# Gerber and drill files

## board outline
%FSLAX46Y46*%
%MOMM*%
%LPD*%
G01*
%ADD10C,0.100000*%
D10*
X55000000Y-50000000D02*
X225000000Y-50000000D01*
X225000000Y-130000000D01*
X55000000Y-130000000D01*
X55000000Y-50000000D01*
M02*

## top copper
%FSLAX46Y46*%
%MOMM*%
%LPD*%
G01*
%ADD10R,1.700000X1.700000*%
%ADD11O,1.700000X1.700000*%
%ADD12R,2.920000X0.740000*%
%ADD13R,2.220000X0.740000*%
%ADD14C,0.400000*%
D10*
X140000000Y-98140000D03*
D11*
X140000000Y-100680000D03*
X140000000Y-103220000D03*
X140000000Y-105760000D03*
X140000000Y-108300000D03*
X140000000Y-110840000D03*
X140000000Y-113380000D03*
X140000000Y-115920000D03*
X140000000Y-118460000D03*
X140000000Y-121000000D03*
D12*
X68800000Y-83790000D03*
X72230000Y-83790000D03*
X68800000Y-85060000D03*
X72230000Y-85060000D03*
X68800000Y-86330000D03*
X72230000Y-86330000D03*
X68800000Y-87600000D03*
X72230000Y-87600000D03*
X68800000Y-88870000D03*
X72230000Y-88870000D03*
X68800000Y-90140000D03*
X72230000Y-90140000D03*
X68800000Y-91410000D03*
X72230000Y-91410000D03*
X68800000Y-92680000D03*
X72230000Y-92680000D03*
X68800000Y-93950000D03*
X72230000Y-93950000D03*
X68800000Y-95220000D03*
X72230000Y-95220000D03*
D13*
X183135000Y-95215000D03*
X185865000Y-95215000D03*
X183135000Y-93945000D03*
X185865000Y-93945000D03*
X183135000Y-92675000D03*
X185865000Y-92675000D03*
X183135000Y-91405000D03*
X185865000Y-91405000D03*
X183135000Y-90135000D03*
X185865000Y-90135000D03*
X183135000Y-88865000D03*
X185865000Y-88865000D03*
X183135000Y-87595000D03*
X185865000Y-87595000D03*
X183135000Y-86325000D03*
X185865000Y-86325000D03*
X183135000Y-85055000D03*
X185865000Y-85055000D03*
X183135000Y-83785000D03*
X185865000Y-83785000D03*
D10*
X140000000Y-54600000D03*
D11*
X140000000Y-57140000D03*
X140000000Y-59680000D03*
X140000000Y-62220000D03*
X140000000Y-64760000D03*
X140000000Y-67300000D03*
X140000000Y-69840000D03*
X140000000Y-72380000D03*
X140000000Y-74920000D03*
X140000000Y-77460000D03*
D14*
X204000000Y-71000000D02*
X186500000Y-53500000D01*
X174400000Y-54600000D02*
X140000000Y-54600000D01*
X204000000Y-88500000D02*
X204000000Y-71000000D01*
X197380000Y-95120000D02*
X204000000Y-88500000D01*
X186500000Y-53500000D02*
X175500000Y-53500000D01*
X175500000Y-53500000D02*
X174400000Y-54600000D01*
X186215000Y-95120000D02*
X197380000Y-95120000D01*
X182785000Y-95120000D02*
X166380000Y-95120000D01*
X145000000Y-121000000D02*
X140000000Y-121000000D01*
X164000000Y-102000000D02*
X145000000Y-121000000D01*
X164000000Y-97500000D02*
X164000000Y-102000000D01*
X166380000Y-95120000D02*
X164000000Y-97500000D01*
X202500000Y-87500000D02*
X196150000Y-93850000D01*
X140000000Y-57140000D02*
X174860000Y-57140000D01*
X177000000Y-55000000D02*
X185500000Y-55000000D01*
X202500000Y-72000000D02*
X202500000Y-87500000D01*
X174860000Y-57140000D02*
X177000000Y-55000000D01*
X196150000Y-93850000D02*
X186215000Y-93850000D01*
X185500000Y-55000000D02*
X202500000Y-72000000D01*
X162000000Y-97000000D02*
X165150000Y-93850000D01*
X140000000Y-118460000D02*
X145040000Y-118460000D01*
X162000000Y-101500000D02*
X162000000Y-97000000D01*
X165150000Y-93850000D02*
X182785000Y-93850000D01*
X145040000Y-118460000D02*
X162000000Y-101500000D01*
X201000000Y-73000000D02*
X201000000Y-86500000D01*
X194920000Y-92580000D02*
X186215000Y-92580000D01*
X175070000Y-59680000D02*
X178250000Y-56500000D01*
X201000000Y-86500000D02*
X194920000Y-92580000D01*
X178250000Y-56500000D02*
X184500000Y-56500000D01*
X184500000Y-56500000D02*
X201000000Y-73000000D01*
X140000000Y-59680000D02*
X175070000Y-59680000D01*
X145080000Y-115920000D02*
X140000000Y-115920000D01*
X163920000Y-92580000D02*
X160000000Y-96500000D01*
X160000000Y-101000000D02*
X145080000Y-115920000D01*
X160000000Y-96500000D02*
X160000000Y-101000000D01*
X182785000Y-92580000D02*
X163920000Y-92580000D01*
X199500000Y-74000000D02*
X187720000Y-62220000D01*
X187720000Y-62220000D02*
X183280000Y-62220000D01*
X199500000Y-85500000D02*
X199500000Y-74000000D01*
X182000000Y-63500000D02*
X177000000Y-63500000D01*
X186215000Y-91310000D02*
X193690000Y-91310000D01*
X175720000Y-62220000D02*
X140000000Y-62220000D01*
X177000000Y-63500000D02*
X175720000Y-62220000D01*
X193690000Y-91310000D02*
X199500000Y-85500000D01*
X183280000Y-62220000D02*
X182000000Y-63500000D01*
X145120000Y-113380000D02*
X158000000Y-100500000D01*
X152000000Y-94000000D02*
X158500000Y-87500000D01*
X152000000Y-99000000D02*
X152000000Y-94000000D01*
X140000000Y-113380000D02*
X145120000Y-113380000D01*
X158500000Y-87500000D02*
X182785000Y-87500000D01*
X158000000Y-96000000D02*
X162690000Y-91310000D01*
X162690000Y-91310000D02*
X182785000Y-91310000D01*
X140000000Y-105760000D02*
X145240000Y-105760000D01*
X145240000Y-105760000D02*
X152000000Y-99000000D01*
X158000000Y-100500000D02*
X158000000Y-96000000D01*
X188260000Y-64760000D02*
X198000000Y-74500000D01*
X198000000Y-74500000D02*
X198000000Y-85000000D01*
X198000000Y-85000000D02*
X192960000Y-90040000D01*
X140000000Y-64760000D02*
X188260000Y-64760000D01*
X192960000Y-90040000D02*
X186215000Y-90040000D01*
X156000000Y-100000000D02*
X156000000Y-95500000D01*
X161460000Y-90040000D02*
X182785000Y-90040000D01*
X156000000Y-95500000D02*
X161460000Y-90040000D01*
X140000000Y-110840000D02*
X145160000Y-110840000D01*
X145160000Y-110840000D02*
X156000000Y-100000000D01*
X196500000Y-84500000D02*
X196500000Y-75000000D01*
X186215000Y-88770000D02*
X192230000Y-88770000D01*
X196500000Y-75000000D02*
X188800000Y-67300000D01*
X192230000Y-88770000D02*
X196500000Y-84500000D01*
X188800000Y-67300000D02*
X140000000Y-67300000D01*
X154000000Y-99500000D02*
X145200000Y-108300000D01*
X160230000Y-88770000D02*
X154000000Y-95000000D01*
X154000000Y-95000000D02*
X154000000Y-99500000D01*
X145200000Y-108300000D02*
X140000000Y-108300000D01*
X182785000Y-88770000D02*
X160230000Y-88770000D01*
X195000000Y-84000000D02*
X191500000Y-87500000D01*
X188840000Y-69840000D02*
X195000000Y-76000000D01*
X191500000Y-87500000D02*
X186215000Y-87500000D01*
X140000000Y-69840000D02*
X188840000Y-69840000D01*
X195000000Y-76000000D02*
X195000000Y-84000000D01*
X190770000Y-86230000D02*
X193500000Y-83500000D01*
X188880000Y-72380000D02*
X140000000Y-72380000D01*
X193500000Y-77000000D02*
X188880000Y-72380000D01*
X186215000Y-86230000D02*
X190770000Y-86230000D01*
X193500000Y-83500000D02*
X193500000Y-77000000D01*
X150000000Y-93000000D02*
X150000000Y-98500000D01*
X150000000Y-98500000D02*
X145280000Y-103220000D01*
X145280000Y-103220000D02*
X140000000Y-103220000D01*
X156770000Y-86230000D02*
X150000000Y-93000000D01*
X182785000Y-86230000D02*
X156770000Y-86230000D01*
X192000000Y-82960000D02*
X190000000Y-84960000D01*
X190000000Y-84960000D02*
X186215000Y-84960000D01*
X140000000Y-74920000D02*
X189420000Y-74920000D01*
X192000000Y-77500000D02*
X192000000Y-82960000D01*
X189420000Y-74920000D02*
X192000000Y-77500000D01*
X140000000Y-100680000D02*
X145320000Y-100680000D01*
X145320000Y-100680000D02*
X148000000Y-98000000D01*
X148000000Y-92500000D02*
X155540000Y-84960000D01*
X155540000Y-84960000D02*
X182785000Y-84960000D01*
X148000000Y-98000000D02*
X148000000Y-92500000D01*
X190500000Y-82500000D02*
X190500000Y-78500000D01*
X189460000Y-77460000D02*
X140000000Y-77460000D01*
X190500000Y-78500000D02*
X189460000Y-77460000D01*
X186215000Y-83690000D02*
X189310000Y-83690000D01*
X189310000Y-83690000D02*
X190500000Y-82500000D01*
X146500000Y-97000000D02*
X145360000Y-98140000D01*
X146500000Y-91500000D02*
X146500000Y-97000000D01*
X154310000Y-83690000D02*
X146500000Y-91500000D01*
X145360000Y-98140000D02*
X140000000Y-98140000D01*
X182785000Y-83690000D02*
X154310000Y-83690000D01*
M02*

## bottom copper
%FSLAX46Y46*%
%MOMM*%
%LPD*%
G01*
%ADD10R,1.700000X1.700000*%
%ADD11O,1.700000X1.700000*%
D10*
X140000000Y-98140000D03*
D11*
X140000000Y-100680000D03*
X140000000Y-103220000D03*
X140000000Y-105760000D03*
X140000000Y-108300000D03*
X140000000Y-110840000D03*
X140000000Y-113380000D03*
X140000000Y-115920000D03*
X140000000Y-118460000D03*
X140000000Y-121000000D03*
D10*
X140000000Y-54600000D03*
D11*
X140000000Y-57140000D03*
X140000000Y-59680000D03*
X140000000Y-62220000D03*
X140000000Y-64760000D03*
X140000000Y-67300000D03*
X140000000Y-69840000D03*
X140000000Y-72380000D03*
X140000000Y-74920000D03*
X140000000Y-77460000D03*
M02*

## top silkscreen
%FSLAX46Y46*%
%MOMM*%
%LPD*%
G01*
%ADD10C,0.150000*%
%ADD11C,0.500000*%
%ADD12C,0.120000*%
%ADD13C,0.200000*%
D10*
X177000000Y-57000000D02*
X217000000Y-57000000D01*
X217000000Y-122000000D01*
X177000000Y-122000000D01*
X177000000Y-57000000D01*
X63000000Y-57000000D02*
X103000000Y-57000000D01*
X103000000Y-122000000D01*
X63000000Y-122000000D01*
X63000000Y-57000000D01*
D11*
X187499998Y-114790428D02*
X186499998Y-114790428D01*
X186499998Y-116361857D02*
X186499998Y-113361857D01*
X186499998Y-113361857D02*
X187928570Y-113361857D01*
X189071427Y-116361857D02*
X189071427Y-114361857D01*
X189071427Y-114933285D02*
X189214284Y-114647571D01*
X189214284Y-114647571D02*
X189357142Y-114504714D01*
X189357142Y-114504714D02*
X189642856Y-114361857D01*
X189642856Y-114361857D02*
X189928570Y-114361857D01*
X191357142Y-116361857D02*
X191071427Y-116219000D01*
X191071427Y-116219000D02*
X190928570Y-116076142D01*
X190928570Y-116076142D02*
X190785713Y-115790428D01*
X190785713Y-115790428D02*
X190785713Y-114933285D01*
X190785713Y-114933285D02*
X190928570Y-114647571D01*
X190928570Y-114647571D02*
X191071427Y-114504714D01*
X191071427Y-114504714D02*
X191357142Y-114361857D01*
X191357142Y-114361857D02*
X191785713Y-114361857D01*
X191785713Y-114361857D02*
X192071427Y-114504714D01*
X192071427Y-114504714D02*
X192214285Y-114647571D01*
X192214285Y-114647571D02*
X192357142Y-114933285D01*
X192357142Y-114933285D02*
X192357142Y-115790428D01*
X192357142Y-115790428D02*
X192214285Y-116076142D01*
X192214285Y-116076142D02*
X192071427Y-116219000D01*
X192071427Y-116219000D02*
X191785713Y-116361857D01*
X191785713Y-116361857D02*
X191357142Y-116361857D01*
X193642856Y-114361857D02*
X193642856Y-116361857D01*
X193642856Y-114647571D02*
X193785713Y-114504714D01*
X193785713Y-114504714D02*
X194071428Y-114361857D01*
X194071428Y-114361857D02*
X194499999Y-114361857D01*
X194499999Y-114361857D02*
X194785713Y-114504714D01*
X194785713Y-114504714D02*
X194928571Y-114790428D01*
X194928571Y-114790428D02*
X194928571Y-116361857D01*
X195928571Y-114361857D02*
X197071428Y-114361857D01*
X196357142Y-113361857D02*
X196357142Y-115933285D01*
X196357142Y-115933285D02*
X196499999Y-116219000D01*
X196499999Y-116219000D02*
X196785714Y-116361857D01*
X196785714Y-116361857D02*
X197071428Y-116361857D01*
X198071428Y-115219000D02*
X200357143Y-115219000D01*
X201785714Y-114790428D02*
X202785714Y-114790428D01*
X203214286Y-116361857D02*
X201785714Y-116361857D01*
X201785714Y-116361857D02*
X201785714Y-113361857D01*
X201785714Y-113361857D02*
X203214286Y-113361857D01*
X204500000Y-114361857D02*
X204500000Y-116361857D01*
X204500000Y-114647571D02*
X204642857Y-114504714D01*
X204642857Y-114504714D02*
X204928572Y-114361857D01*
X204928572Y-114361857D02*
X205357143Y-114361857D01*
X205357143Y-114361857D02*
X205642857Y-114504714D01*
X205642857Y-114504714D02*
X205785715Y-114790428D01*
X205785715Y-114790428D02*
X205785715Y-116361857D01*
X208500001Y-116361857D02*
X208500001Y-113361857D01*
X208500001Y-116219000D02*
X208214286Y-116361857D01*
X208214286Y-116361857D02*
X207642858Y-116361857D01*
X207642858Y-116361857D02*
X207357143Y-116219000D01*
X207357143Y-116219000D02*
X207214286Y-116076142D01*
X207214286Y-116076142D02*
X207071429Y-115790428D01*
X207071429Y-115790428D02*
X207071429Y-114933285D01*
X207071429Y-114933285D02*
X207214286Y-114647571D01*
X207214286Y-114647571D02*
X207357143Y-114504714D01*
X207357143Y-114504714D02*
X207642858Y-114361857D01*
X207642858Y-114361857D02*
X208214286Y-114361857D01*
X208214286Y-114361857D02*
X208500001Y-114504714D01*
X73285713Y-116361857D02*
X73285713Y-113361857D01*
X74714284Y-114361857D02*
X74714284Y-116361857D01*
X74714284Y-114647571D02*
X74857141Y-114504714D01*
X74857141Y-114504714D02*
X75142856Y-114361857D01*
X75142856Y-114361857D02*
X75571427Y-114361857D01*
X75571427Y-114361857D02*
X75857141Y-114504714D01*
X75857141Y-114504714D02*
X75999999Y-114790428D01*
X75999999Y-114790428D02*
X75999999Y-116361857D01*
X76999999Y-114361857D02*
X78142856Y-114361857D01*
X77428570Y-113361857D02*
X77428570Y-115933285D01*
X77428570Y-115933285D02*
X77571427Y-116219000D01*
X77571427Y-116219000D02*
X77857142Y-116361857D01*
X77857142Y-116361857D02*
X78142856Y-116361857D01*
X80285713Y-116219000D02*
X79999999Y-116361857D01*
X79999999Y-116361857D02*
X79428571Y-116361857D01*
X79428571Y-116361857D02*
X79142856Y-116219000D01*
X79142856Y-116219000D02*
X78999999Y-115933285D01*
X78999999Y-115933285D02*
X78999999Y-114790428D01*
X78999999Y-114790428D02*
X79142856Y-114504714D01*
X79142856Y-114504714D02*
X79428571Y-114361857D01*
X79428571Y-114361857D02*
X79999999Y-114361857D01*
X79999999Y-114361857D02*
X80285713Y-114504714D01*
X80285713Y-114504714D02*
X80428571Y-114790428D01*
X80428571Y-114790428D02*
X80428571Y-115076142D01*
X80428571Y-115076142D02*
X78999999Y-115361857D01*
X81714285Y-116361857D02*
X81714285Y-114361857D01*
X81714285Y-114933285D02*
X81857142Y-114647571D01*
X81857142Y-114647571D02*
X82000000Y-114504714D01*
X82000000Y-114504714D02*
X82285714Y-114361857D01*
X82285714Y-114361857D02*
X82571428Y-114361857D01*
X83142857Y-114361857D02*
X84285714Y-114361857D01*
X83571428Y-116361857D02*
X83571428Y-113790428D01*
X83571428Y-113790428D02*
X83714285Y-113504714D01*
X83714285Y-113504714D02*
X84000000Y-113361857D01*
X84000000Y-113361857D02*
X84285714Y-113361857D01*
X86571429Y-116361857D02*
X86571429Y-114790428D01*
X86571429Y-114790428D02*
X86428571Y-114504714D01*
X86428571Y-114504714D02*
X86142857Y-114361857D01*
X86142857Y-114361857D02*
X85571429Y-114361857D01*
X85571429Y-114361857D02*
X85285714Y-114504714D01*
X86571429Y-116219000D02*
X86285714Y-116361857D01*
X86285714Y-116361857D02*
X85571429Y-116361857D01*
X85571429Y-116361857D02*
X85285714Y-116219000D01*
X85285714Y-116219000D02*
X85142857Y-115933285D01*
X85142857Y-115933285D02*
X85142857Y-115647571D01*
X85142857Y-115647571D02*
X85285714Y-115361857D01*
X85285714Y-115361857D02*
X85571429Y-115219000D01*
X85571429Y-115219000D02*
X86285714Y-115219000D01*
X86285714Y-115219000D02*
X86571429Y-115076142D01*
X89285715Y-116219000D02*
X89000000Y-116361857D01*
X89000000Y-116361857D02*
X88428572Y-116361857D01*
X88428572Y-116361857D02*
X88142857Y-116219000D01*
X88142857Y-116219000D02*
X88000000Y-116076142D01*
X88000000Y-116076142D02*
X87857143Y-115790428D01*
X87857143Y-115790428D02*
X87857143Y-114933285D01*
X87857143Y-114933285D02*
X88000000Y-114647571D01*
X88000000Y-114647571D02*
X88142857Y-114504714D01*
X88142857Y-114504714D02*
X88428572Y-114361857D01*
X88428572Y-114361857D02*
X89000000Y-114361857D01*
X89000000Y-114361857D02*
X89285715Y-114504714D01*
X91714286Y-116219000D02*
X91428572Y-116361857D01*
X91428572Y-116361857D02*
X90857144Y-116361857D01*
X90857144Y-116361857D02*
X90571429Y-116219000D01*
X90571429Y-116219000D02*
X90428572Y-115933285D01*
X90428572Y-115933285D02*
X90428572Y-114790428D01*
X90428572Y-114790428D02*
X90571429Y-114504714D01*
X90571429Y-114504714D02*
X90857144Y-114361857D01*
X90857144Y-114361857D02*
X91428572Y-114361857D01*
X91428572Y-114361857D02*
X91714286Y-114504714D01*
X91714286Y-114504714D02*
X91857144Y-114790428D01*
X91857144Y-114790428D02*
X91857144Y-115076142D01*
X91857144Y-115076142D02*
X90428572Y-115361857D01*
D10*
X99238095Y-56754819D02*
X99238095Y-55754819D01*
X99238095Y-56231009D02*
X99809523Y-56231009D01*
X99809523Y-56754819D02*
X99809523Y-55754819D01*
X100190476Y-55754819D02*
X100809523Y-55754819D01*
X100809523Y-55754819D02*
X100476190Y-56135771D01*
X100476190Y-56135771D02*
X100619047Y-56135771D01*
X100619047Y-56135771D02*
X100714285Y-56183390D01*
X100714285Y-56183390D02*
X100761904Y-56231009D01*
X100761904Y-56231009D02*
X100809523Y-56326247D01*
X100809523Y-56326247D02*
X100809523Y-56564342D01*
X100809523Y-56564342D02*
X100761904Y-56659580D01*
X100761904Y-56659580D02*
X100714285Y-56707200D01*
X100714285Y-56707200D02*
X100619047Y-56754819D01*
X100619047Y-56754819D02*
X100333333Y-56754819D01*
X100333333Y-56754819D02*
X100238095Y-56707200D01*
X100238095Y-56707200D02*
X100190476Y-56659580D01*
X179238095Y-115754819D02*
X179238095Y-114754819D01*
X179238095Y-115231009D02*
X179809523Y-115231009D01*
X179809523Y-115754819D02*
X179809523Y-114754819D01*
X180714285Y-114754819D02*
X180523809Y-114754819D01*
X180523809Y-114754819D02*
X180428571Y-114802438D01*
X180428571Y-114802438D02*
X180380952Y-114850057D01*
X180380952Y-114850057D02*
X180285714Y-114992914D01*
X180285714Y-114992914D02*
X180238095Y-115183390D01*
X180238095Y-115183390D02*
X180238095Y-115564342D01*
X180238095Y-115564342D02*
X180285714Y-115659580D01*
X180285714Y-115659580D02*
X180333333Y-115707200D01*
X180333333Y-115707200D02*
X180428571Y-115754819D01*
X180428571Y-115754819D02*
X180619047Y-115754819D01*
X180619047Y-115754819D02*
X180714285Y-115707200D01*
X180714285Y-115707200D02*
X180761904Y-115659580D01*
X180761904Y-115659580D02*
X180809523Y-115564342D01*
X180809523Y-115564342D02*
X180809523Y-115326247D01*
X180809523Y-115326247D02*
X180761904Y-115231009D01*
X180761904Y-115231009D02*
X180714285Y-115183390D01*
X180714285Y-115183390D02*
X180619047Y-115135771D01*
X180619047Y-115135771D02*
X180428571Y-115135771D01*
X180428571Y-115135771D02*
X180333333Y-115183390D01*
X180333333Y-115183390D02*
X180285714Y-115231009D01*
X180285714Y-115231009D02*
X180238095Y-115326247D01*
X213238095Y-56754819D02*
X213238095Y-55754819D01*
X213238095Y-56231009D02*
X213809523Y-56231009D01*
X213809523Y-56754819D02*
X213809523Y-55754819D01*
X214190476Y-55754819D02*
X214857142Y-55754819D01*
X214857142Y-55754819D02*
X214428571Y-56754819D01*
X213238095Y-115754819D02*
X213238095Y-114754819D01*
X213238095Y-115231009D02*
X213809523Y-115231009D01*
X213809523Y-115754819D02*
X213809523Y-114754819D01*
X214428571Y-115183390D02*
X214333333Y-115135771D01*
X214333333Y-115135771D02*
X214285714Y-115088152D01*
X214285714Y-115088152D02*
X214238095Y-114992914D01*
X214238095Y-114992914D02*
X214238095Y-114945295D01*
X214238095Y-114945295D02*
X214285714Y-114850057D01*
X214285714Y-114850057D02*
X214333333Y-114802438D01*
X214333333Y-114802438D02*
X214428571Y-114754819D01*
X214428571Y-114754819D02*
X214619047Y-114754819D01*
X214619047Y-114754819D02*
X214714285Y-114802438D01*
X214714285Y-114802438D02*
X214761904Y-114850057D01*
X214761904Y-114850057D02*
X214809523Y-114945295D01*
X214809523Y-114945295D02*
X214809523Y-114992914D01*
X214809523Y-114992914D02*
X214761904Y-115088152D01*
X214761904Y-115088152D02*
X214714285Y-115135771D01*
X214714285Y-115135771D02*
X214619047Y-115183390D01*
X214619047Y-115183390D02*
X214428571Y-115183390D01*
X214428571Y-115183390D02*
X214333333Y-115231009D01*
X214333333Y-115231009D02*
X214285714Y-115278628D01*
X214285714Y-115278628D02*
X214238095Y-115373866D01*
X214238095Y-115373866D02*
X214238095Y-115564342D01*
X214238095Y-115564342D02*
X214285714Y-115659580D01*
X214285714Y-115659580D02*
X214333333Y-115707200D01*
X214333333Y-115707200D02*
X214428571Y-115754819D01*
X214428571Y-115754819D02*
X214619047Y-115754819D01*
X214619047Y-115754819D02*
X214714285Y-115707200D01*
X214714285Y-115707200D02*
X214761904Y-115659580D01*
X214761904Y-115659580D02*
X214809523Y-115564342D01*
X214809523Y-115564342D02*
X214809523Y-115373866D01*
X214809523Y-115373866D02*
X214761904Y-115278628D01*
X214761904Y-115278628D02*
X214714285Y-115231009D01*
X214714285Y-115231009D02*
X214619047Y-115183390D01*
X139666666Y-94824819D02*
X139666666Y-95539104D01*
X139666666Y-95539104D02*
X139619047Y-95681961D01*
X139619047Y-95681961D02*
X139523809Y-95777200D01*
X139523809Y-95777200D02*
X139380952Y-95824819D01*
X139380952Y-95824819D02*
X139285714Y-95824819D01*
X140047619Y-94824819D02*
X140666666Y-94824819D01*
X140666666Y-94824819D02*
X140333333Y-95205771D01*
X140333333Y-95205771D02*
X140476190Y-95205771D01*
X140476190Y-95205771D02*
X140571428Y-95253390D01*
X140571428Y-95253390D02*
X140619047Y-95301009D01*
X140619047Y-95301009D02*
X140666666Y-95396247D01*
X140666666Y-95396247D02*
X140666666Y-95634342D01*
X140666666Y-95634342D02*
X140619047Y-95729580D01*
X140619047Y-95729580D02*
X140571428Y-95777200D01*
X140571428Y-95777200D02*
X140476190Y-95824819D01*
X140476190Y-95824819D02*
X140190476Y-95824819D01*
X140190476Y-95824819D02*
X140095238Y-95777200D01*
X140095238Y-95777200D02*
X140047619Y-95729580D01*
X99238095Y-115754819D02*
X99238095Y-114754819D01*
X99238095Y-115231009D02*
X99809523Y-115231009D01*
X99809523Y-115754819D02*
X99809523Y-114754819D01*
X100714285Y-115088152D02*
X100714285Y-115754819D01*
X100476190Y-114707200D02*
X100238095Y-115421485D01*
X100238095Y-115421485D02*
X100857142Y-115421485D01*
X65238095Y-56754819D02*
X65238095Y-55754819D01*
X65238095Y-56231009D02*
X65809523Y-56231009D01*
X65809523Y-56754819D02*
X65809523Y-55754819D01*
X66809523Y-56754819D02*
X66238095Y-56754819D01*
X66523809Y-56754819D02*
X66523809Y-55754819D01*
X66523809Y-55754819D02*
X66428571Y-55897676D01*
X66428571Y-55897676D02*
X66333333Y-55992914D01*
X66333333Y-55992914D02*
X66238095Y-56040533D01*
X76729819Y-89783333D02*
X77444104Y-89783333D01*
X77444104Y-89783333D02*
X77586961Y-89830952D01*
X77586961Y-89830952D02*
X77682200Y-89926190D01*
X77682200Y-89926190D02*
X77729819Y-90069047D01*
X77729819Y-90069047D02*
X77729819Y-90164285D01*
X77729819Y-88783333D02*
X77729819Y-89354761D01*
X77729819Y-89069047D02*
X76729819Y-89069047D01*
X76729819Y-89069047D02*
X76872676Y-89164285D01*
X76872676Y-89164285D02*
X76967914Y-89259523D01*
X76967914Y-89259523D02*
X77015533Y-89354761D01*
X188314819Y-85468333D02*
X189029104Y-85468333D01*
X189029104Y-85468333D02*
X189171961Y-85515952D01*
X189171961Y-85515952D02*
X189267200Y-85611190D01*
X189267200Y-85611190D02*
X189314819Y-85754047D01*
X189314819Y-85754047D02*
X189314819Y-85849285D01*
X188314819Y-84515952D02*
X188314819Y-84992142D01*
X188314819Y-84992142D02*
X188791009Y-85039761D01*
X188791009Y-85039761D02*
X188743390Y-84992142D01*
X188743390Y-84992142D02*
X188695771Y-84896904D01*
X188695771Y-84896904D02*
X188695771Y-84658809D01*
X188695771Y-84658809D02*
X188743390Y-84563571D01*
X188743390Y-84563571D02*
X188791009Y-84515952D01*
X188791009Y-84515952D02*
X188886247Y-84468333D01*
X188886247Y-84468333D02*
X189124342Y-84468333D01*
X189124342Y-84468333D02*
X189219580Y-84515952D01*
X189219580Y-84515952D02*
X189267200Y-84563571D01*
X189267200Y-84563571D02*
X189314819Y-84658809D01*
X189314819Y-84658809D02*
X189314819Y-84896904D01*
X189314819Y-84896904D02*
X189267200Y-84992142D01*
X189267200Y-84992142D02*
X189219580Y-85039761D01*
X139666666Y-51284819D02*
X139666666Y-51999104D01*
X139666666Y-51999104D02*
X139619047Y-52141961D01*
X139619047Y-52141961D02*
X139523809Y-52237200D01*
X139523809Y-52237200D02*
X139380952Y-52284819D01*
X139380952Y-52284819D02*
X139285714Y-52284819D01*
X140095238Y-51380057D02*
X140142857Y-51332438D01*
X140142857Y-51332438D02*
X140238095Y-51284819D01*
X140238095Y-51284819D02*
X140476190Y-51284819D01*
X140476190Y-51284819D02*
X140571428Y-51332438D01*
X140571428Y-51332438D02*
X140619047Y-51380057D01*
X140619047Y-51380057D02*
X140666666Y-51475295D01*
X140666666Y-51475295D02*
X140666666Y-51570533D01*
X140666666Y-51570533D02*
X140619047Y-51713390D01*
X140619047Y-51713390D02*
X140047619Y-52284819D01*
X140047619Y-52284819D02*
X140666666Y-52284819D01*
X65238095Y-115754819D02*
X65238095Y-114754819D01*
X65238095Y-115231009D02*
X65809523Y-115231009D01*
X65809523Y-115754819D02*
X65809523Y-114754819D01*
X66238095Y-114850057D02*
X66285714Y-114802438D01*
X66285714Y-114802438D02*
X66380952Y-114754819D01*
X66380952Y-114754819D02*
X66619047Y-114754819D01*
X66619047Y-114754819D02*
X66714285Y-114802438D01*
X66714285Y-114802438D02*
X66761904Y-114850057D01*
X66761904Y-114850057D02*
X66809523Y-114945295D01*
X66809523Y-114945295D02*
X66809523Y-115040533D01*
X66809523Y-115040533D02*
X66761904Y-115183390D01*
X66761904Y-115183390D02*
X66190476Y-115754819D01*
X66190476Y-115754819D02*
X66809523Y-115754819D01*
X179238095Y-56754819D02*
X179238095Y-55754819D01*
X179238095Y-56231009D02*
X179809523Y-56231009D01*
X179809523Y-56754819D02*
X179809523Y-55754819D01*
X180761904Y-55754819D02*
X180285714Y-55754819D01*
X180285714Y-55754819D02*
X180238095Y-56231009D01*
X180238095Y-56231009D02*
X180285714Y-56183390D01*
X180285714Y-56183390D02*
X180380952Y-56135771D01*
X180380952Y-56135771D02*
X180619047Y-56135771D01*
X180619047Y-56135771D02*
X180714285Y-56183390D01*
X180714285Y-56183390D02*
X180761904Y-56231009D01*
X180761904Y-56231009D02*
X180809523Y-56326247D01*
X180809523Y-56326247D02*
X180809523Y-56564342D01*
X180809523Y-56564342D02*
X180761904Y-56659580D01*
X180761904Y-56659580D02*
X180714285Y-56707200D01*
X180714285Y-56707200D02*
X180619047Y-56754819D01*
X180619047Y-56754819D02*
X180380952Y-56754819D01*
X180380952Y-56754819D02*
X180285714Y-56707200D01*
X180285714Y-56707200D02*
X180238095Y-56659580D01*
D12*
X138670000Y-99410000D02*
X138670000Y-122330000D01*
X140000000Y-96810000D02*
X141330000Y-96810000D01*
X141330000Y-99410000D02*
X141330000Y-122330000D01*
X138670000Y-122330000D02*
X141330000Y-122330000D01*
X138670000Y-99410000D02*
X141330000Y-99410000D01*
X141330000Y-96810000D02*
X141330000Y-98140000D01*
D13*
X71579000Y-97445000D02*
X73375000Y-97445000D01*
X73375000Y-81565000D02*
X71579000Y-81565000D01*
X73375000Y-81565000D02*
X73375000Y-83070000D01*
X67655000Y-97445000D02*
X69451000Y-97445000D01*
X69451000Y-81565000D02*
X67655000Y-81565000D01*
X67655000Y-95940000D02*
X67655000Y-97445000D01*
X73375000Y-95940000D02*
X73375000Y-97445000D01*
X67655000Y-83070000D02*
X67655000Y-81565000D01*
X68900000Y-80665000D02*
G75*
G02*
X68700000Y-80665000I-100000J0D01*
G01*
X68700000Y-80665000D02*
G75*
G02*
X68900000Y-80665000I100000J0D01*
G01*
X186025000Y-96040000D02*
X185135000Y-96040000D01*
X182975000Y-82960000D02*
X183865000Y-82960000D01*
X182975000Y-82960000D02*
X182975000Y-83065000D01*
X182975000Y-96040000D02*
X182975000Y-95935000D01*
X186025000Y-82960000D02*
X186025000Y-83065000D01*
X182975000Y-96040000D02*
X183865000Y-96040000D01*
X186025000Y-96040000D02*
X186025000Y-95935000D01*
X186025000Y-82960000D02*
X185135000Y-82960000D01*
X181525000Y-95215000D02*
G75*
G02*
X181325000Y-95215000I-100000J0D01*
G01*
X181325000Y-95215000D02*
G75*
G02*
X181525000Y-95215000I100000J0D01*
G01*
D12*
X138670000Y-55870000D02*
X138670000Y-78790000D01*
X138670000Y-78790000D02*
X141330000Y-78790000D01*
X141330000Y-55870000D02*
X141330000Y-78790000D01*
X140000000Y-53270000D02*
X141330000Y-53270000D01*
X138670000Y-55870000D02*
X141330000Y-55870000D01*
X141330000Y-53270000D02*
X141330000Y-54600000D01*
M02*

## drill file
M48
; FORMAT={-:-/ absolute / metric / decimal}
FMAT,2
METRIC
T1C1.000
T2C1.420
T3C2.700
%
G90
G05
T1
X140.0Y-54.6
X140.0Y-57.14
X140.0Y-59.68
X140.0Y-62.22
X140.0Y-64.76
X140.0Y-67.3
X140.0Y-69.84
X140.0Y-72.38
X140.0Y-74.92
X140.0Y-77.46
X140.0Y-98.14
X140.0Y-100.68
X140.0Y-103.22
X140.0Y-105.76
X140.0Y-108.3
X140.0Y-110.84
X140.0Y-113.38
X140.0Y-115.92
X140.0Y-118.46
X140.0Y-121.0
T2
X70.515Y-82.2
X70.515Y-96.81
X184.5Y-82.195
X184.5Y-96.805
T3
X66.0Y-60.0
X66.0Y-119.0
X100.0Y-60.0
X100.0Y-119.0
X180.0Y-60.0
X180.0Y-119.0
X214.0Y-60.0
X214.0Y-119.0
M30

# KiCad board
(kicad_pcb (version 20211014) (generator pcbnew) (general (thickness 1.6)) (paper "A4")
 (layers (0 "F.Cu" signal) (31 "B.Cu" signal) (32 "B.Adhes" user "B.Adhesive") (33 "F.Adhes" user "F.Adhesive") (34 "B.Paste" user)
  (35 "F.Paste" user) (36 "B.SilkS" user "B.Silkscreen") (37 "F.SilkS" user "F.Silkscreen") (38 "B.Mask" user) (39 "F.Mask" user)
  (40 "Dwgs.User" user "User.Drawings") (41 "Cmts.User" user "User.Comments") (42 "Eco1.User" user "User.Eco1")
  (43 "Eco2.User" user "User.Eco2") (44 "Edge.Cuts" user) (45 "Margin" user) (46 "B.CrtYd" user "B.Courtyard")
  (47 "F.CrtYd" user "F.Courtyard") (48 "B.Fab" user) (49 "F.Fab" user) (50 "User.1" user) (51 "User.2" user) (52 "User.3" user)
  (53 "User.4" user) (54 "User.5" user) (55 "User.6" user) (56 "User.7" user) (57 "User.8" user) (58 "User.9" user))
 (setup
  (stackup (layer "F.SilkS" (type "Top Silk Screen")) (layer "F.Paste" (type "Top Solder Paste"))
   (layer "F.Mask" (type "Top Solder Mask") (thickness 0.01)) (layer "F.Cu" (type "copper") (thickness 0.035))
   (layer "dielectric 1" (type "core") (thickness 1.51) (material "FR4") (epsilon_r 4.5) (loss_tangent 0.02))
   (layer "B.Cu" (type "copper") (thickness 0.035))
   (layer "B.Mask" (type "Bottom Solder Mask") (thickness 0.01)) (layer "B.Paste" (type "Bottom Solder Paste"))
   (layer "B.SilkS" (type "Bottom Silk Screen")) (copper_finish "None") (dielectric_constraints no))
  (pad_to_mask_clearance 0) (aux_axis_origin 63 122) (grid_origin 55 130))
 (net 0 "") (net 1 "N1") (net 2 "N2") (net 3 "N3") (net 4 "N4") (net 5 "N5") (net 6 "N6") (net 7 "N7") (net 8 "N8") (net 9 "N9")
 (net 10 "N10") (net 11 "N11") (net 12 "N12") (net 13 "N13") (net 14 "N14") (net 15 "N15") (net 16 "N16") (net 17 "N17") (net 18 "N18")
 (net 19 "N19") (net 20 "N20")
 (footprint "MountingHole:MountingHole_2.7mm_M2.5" (layer "F.Cu") (at 100 60)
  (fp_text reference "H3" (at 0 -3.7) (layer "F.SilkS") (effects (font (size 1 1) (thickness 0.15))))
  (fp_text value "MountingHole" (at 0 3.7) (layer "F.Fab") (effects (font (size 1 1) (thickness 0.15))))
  (pad "" np_thru_hole circle (at 0 0) (size 2.7 2.7) (drill 2.7) (layers *.Cu *.Mask)))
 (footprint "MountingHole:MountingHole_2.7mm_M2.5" (layer "F.Cu") (at 180 119)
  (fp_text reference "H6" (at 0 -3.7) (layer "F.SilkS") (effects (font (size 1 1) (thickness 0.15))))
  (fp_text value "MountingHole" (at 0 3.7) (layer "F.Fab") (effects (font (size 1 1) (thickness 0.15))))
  (pad "" np_thru_hole circle (at 0 0) (size 2.7 2.7) (drill 2.7) (layers *.Cu *.Mask)))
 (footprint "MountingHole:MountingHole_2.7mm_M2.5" (layer "F.Cu") (at 214 60)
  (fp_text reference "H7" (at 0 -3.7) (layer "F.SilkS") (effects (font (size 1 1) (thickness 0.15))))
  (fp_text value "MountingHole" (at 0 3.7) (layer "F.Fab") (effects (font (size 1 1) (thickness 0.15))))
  (pad "" np_thru_hole circle (at 0 0) (size 2.7 2.7) (drill 2.7) (layers *.Cu *.Mask)))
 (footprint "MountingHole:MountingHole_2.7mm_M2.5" (layer "F.Cu") (at 214 119)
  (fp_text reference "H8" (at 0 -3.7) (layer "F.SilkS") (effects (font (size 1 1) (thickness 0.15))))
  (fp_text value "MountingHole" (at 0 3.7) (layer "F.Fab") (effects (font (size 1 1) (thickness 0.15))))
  (pad "" np_thru_hole circle (at 0 0) (size 2.7 2.7) (drill 2.7) (layers *.Cu *.Mask)))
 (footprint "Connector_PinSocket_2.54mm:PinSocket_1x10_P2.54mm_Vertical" (layer "F.Cu") (at 140 98.14)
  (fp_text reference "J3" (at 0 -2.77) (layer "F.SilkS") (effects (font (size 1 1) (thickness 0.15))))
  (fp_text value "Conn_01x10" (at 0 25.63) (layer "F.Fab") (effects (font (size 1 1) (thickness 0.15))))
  (fp_line (start -1.33 1.27) (end -1.33 24.19) (layer "F.SilkS") (width 0.12))
  (fp_line (start 0 -1.33) (end 1.33 -1.33) (layer "F.SilkS") (width 0.12))
  (fp_line (start 1.33 1.27) (end 1.33 24.19) (layer "F.SilkS") (width 0.12))
  (fp_line (start -1.33 24.19) (end 1.33 24.19) (layer "F.SilkS") (width 0.12))
  (fp_line (start -1.33 1.27) (end 1.33 1.27) (layer "F.SilkS") (width 0.12))
  (fp_line (start 1.33 -1.33) (end 1.33 0) (layer "F.SilkS") (width 0.12))
  (pad "1" thru_hole rect (at 0 0) (size 1.7 1.7) (drill 1) (layers *.Cu *.Mask) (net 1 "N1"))
  (pad "2" thru_hole oval (at 0 2.54) (size 1.7 1.7) (drill 1) (layers *.Cu *.Mask) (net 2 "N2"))
  (pad "3" thru_hole oval (at 0 5.08) (size 1.7 1.7) (drill 1) (layers *.Cu *.Mask) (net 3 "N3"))
  (pad "4" thru_hole oval (at 0 7.62) (size 1.7 1.7) (drill 1) (layers *.Cu *.Mask) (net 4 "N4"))
  (pad "5" thru_hole oval (at 0 10.16) (size 1.7 1.7) (drill 1) (layers *.Cu *.Mask) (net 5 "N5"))
  (pad "6" thru_hole oval (at 0 12.7) (size 1.7 1.7) (drill 1) (layers *.Cu *.Mask) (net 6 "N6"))
  (pad "7" thru_hole oval (at 0 15.24) (size 1.7 1.7) (drill 1) (layers *.Cu *.Mask) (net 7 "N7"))
  (pad "8" thru_hole oval (at 0 17.78) (size 1.7 1.7) (drill 1) (layers *.Cu *.Mask) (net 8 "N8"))
  (pad "9" thru_hole oval (at 0 20.32) (size 1.7 1.7) (drill 1) (layers *.Cu *.Mask) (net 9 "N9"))
  (pad "10" thru_hole oval (at 0 22.86) (size 1.7 1.7) (drill 1) (layers *.Cu *.Mask) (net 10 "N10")))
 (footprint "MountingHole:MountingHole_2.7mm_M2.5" (layer "F.Cu") (at 100 119)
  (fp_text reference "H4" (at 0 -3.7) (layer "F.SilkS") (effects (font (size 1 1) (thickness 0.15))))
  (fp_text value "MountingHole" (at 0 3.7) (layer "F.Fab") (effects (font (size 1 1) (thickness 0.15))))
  (pad "" np_thru_hole circle (at 0 0) (size 2.7 2.7) (drill 2.7) (layers *.Cu *.Mask)))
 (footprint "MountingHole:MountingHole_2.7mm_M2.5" (layer "F.Cu") (at 66 60)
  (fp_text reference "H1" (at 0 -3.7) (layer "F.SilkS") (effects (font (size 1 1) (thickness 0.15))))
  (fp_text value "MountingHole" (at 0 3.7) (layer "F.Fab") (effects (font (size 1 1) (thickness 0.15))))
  (pad "" np_thru_hole circle (at 0 0) (size 2.7 2.7) (drill 2.7) (layers *.Cu *.Mask)))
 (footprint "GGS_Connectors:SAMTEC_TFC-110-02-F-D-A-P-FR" (layer "F.Cu") (at 70.5 89.5 -90)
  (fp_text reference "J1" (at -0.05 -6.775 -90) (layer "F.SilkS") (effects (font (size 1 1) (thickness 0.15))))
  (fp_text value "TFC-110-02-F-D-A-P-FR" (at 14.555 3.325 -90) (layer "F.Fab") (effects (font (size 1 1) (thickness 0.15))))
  (fp_line (start 7.945 -1.079) (end 7.945 -2.875) (layer "F.SilkS") (width 0.2))
  (fp_line (start -7.935 -2.875) (end -7.935 -1.079) (layer "F.SilkS") (width 0.2))
  (fp_line (start -7.935 -2.875) (end -6.43 -2.875) (layer "F.SilkS") (width 0.2))
  (fp_line (start 7.945 2.845) (end 7.945 1.049) (layer "F.SilkS") (width 0.2))
  (fp_line (start -7.935 1.049) (end -7.935 2.845) (layer "F.SilkS") (width 0.2))
  (fp_line (start 6.44 2.845) (end 7.945 2.845) (layer "F.SilkS") (width 0.2))
  (fp_line (start 6.44 -2.875) (end 7.945 -2.875) (layer "F.SilkS") (width 0.2))
  (fp_line (start -6.43 2.845) (end -7.935 2.845) (layer "F.SilkS") (width 0.2))
  (fp_circle (center -8.835 1.7) (end -8.735 1.7) (layer "F.SilkS") (width 0.2) (fill none))
  (pad "" np_thru_hole circle (at -7.3 -0.015 270) (size 1.42 1.42) (drill 1.42) (layers *.Cu *.Mask))
  (pad "" np_thru_hole circle (at 7.31 -0.015 270) (size 1.42 1.42) (drill 1.42) (layers *.Cu *.Mask))
  (pad "01" smd rect (at -5.71 1.7 270) (size 0.74 2.92) (layers "F.Cu" "F.Paste" "F.Mask") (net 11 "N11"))
  (pad "02" smd rect (at -5.71 -1.73 270) (size 0.74 2.92) (layers "F.Cu" "F.Paste" "F.Mask") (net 10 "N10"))
  (pad "03" smd rect (at -4.44 1.7 270) (size 0.74 2.92) (layers "F.Cu" "F.Paste" "F.Mask") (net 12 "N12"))
  (pad "04" smd rect (at -4.44 -1.73 270) (size 0.74 2.92) (layers "F.Cu" "F.Paste" "F.Mask") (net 9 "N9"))
  (pad "05" smd rect (at -3.17 1.7 270) (size 0.74 2.92) (layers "F.Cu" "F.Paste" "F.Mask") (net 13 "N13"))
  (pad "06" smd rect (at -3.17 -1.73 270) (size 0.74 2.92) (layers "F.Cu" "F.Paste" "F.Mask") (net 8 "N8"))
  (pad "07" smd rect (at -1.9 1.7 270) (size 0.74 2.92) (layers "F.Cu" "F.Paste" "F.Mask") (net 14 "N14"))
  (pad "08" smd rect (at -1.9 -1.73 270) (size 0.74 2.92) (layers "F.Cu" "F.Paste" "F.Mask") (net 7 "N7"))
  (pad "09" smd rect (at -0.63 1.7 270) (size 0.74 2.92) (layers "F.Cu" "F.Paste" "F.Mask") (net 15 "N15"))
  (pad "10" smd rect (at -0.63 -1.73 270) (size 0.74 2.92) (layers "F.Cu" "F.Paste" "F.Mask") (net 6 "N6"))
  (pad "11" smd rect (at 0.64 1.7 270) (size 0.74 2.92) (layers "F.Cu" "F.Paste" "F.Mask") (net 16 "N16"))
  (pad "12" smd rect (at 0.64 -1.73 270) (size 0.74 2.92) (layers "F.Cu" "F.Paste" "F.Mask") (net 5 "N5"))
  (pad "13" smd rect (at 1.91 1.7 270) (size 0.74 2.92) (layers "F.Cu" "F.Paste" "F.Mask") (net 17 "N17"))
  (pad "14" smd rect (at 1.91 -1.73 270) (size 0.74 2.92) (layers "F.Cu" "F.Paste" "F.Mask") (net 4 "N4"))
  (pad "15" smd rect (at 3.18 1.7 270) (size 0.74 2.92) (layers "F.Cu" "F.Paste" "F.Mask") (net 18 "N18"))
  (pad "16" smd rect (at 3.18 -1.73 270) (size 0.74 2.92) (layers "F.Cu" "F.Paste" "F.Mask") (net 3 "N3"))
  (pad "17" smd rect (at 4.45 1.7 270) (size 0.74 2.92) (layers "F.Cu" "F.Paste" "F.Mask") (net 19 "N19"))
  (pad "18" smd rect (at 4.45 -1.73 270) (size 0.74 2.92) (layers "F.Cu" "F.Paste" "F.Mask") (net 2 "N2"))
  (pad "19" smd rect (at 5.72 1.7 270) (size 0.74 2.92) (layers "F.Cu" "F.Paste" "F.Mask") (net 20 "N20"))
  (pad "20" smd rect (at 5.72 -1.73 270) (size 0.74 2.92) (layers "F.Cu" "F.Paste" "F.Mask") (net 1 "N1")))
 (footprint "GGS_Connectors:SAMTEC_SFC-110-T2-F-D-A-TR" (layer "F.Cu") (at 184.5 89.5 -90)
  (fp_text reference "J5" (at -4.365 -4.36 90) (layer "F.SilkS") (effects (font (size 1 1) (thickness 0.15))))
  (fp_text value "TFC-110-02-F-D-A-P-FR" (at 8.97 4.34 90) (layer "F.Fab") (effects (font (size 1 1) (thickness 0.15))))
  (fp_line (start 6.54 -1.525) (end 6.54 -0.635) (layer "F.SilkS") (width 0.2))
  (fp_line (start -6.54 1.525) (end -6.54 0.635) (layer "F.SilkS") (width 0.2))
  (fp_line (start -6.54 1.525) (end -6.435 1.525) (layer "F.SilkS") (width 0.2))
  (fp_line (start 6.54 1.525) (end 6.435 1.525) (layer "F.SilkS") (width 0.2))
  (fp_line (start -6.54 -1.525) (end -6.435 -1.525) (layer "F.SilkS") (width 0.2))
  (fp_line (start 6.54 1.525) (end 6.54 0.635) (layer "F.SilkS") (width 0.2))
  (fp_line (start 6.54 -1.525) (end 6.435 -1.525) (layer "F.SilkS") (width 0.2))
  (fp_line (start -6.54 -1.525) (end -6.54 -0.635) (layer "F.SilkS") (width 0.2))
  (fp_circle (center 5.715 3.075) (end 5.815 3.075) (layer "F.SilkS") (width 0.2) (fill none))
  (pad "" np_thru_hole circle (at -7.305 0 270) (size 1.42 1.42) (drill 1.42) (layers *.Cu *.Mask))
  (pad "" np_thru_hole circle (at 7.305 0 270) (size 1.42 1.42) (drill 1.42) (layers *.Cu *.Mask))
  (pad "01" smd rect (at 5.715 1.365 270) (size 0.74 2.22) (layers "F.Cu" "F.Paste" "F.Mask") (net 11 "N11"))
  (pad "02" smd rect (at 5.715 -1.365 270) (size 0.74 2.22) (layers "F.Cu" "F.Paste" "F.Mask") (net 10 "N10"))
  (pad "03" smd rect (at 4.445 1.365 270) (size 0.74 2.22) (layers "F.Cu" "F.Paste" "F.Mask") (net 12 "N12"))
  (pad "04" smd rect (at 4.445 -1.365 270) (size 0.74 2.22) (layers "F.Cu" "F.Paste" "F.Mask") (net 9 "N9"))
  (pad "05" smd rect (at 3.175 1.365 270) (size 0.74 2.22) (layers "F.Cu" "F.Paste" "F.Mask") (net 13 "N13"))
  (pad "06" smd rect (at 3.175 -1.365 270) (size 0.74 2.22) (layers "F.Cu" "F.Paste" "F.Mask") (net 8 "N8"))
  (pad "07" smd rect (at 1.905 1.365 270) (size 0.74 2.22) (layers "F.Cu" "F.Paste" "F.Mask") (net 14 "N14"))
  (pad "08" smd rect (at 1.905 -1.365 270) (size 0.74 2.22) (layers "F.Cu" "F.Paste" "F.Mask") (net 7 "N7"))
  (pad "09" smd rect (at 0.635 1.365 270) (size 0.74 2.22) (layers "F.Cu" "F.Paste" "F.Mask") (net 15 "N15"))
  (pad "10" smd rect (at 0.635 -1.365 270) (size 0.74 2.22) (layers "F.Cu" "F.Paste" "F.Mask") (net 6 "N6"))
  (pad "11" smd rect (at -0.635 1.365 270) (size 0.74 2.22) (layers "F.Cu" "F.Paste" "F.Mask") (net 16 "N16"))
  (pad "12" smd rect (at -0.635 -1.365 270) (size 0.74 2.22) (layers "F.Cu" "F.Paste" "F.Mask") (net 5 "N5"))
  (pad "13" smd rect (at -1.905 1.365 270) (size 0.74 2.22) (layers "F.Cu" "F.Paste" "F.Mask") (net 17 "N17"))
  (pad "14" smd rect (at -1.905 -1.365 270) (size 0.74 2.22) (layers "F.Cu" "F.Paste" "F.Mask") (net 4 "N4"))
  (pad "15" smd rect (at -3.175 1.365 270) (size 0.74 2.22) (layers "F.Cu" "F.Paste" "F.Mask") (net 18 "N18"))
  (pad "16" smd rect (at -3.175 -1.365 270) (size 0.74 2.22) (layers "F.Cu" "F.Paste" "F.Mask") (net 3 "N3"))
  (pad "17" smd rect (at -4.445 1.365 270) (size 0.74 2.22) (layers "F.Cu" "F.Paste" "F.Mask") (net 19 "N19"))
  (pad "18" smd rect (at -4.445 -1.365 270) (size 0.74 2.22) (layers "F.Cu" "F.Paste" "F.Mask") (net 2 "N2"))
  (pad "19" smd rect (at -5.715 1.365 270) (size 0.74 2.22) (layers "F.Cu" "F.Paste" "F.Mask") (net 20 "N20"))
  (pad "20" smd rect (at -5.715 -1.365 270) (size 0.74 2.22) (layers "F.Cu" "F.Paste" "F.Mask") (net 1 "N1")))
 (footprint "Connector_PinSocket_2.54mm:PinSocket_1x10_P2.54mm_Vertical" (layer "F.Cu") (at 140 54.6)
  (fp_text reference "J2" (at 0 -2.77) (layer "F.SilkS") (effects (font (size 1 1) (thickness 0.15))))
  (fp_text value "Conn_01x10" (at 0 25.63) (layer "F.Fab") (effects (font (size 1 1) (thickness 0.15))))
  (fp_line (start -1.33 1.27) (end -1.33 24.19) (layer "F.SilkS") (width 0.12))
  (fp_line (start -1.33 24.19) (end 1.33 24.19) (layer "F.SilkS") (width 0.12))
  (fp_line (start 1.33 1.27) (end 1.33 24.19) (layer "F.SilkS") (width 0.12))
  (fp_line (start 0 -1.33) (end 1.33 -1.33) (layer "F.SilkS") (width 0.12))
  (fp_line (start -1.33 1.27) (end 1.33 1.27) (layer "F.SilkS") (width 0.12))
  (fp_line (start 1.33 -1.33) (end 1.33 0) (layer "F.SilkS") (width 0.12))
  (pad "1" thru_hole rect (at 0 0) (size 1.7 1.7) (drill 1) (layers *.Cu *.Mask) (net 11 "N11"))
  (pad "2" thru_hole oval (at 0 2.54) (size 1.7 1.7) (drill 1) (layers *.Cu *.Mask) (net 12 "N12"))
  (pad "3" thru_hole oval (at 0 5.08) (size 1.7 1.7) (drill 1) (layers *.Cu *.Mask) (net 13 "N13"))
  (pad "4" thru_hole oval (at 0 7.62) (size 1.7 1.7) (drill 1) (layers *.Cu *.Mask) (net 14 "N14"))
  (pad "5" thru_hole oval (at 0 10.16) (size 1.7 1.7) (drill 1) (layers *.Cu *.Mask) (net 15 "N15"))
  (pad "6" thru_hole oval (at 0 12.7) (size 1.7 1.7) (drill 1) (layers *.Cu *.Mask) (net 16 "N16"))
  (pad "7" thru_hole oval (at 0 15.24) (size 1.7 1.7) (drill 1) (layers *.Cu *.Mask) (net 17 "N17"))
  (pad "8" thru_hole oval (at 0 17.78) (size 1.7 1.7) (drill 1) (layers *.Cu *.Mask) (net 18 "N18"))
  (pad "9" thru_hole oval (at 0 20.32) (size 1.7 1.7) (drill 1) (layers *.Cu *.Mask) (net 19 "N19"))
  (pad "10" thru_hole oval (at 0 22.86) (size 1.7 1.7) (drill 1) (layers *.Cu *.Mask) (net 20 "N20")))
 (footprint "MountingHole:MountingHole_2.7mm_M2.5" (layer "F.Cu") (at 66 119)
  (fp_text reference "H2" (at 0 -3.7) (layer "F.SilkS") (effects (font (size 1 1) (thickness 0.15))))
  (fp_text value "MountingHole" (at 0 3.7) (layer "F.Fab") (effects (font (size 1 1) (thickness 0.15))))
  (pad "" np_thru_hole circle (at 0 0) (size 2.7 2.7) (drill 2.7) (layers *.Cu *.Mask)))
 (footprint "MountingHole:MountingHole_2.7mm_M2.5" (layer "F.Cu") (at 180 60)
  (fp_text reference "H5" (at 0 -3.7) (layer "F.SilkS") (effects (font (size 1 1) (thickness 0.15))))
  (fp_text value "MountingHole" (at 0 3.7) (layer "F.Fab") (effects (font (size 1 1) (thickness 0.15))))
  (pad "" np_thru_hole circle (at 0 0) (size 2.7 2.7) (drill 2.7) (layers *.Cu *.Mask)))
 (gr_rect (start 177 57) (end 217 122) (layer "F.SilkS") (width 0.15) (fill none))
 (gr_rect (start 63 57) (end 103 122) (layer "F.SilkS") (width 0.15) (fill none))
 (gr_rect (start 55 50) (end 225 130) (layer "Edge.Cuts") (width 0.1) (fill none))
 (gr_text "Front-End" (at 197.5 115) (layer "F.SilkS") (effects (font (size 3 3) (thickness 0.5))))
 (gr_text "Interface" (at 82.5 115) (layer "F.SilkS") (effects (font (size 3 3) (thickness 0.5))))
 (segment (start 204 71) (end 186.5 53.5) (width 0.4) (layer "F.Cu") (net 11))
 (segment (start 174.4 54.6) (end 140 54.6) (width 0.4) (layer "F.Cu") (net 11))
 (segment (start 204 88.5) (end 204 71) (width 0.4) (layer "F.Cu") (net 11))
 (segment (start 197.38 95.12) (end 204 88.5) (width 0.4) (layer "F.Cu") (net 11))
 (segment (start 186.5 53.5) (end 175.5 53.5) (width 0.4) (layer "F.Cu") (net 11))
 (segment (start 175.5 53.5) (end 174.4 54.6) (width 0.4) (layer "F.Cu") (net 11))
 (segment (start 186.215 95.12) (end 197.38 95.12) (width 0.4) (layer "F.Cu") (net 11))
 (segment (start 182.785 95.12) (end 166.38 95.12) (width 0.4) (layer "F.Cu") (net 10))
 (segment (start 145 121) (end 140 121) (width 0.4) (layer "F.Cu") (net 10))
 (segment (start 164 102) (end 145 121) (width 0.4) (layer "F.Cu") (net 10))
 (segment (start 164 97.5) (end 164 102) (width 0.4) (layer "F.Cu") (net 10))
 (segment (start 166.38 95.12) (end 164 97.5) (width 0.4) (layer "F.Cu") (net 10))
 (segment (start 202.5 87.5) (end 196.15 93.85) (width 0.4) (layer "F.Cu") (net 12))
 (segment (start 140 57.14) (end 174.86 57.14) (width 0.4) (layer "F.Cu") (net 12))
 (segment (start 177 55) (end 185.5 55) (width 0.4) (layer "F.Cu") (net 12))
 (segment (start 202.5 72) (end 202.5 87.5) (width 0.4) (layer "F.Cu") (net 12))
 (segment (start 174.86 57.14) (end 177 55) (width 0.4) (layer "F.Cu") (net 12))
 (segment (start 196.15 93.85) (end 186.215 93.85) (width 0.4) (layer "F.Cu") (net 12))
 (segment (start 185.5 55) (end 202.5 72) (width 0.4) (layer "F.Cu") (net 12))
 (segment (start 162 97) (end 165.15 93.85) (width 0.4) (layer "F.Cu") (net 9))
 (segment (start 140 118.46) (end 145.04 118.46) (width 0.4) (layer "F.Cu") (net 9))
 (segment (start 162 101.5) (end 162 97) (width 0.4) (layer "F.Cu") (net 9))
 (segment (start 165.15 93.85) (end 182.785 93.85) (width 0.4) (layer "F.Cu") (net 9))
 (segment (start 145.04 118.46) (end 162 101.5) (width 0.4) (layer "F.Cu") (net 9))
 (segment (start 201 73) (end 201 86.5) (width 0.4) (layer "F.Cu") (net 13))
 (segment (start 194.92 92.58) (end 186.215 92.58) (width 0.4) (layer "F.Cu") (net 13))
 (segment (start 175.07 59.68) (end 178.25 56.5) (width 0.4) (layer "F.Cu") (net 13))
 (segment (start 201 86.5) (end 194.92 92.58) (width 0.4) (layer "F.Cu") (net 13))
 (segment (start 178.25 56.5) (end 184.5 56.5) (width 0.4) (layer "F.Cu") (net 13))
 (segment (start 184.5 56.5) (end 201 73) (width 0.4) (layer "F.Cu") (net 13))
 (segment (start 140 59.68) (end 175.07 59.68) (width 0.4) (layer "F.Cu") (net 13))
 (segment (start 145.08 115.92) (end 140 115.92) (width 0.4) (layer "F.Cu") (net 8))
 (segment (start 163.92 92.58) (end 160 96.5) (width 0.4) (layer "F.Cu") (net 8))
 (segment (start 160 101) (end 145.08 115.92) (width 0.4) (layer "F.Cu") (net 8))
 (segment (start 160 96.5) (end 160 101) (width 0.4) (layer "F.Cu") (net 8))
 (segment (start 182.785 92.58) (end 163.92 92.58) (width 0.4) (layer "F.Cu") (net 8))
 (segment (start 199.5 74) (end 187.72 62.22) (width 0.4) (layer "F.Cu") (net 14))
 (segment (start 187.72 62.22) (end 183.28 62.22) (width 0.4) (layer "F.Cu") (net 14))
 (segment (start 199.5 85.5) (end 199.5 74) (width 0.4) (layer "F.Cu") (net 14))
 (segment (start 182 63.5) (end 177 63.5) (width 0.4) (layer "F.Cu") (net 14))
 (segment (start 186.215 91.31) (end 193.69 91.31) (width 0.4) (layer "F.Cu") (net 14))
 (segment (start 175.72 62.22) (end 140 62.22) (width 0.4) (layer "F.Cu") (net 14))
 (segment (start 177 63.5) (end 175.72 62.22) (width 0.4) (layer "F.Cu") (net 14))
 (segment (start 193.69 91.31) (end 199.5 85.5) (width 0.4) (layer "F.Cu") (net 14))
 (segment (start 183.28 62.22) (end 182 63.5) (width 0.4) (layer "F.Cu") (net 14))
 (segment (start 145.12 113.38) (end 158 100.5) (width 0.4) (layer "F.Cu") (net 7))
 (segment (start 152 94) (end 158.5 87.5) (width 0.4) (layer "F.Cu") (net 7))
 (segment (start 152 99) (end 152 94) (width 0.4) (layer "F.Cu") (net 7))
 (segment (start 140 113.38) (end 145.12 113.38) (width 0.4) (layer "F.Cu") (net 7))
 (segment (start 158.5 87.5) (end 182.785 87.5) (width 0.4) (layer "F.Cu") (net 7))
 (segment (start 158 96) (end 162.69 91.31) (width 0.4) (layer "F.Cu") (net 7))
 (segment (start 162.69 91.31) (end 182.785 91.31) (width 0.4) (layer "F.Cu") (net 7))
 (segment (start 140 105.76) (end 145.24 105.76) (width 0.4) (layer "F.Cu") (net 7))
 (segment (start 145.24 105.76) (end 152 99) (width 0.4) (layer "F.Cu") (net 7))
 (segment (start 158 100.5) (end 158 96) (width 0.4) (layer "F.Cu") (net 7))
 (segment (start 188.26 64.76) (end 198 74.5) (width 0.4) (layer "F.Cu") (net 15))
 (segment (start 198 74.5) (end 198 85) (width 0.4) (layer "F.Cu") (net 15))
 (segment (start 198 85) (end 192.96 90.04) (width 0.4) (layer "F.Cu") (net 15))
 (segment (start 140 64.76) (end 188.26 64.76) (width 0.4) (layer "F.Cu") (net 15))
 (segment (start 192.96 90.04) (end 186.215 90.04) (width 0.4) (layer "F.Cu") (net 15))
 (segment (start 156 100) (end 156 95.5) (width 0.4) (layer "F.Cu") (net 6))
 (segment (start 161.46 90.04) (end 182.785 90.04) (width 0.4) (layer "F.Cu") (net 6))
 (segment (start 156 95.5) (end 161.46 90.04) (width 0.4) (layer "F.Cu") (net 6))
 (segment (start 140 110.84) (end 145.16 110.84) (width 0.4) (layer "F.Cu") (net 6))
 (segment (start 145.16 110.84) (end 156 100) (width 0.4) (layer "F.Cu") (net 6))
 (segment (start 196.5 84.5) (end 196.5 75) (width 0.4) (layer "F.Cu") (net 16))
 (segment (start 186.215 88.77) (end 192.23 88.77) (width 0.4) (layer "F.Cu") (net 16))
 (segment (start 196.5 75) (end 188.8 67.3) (width 0.4) (layer "F.Cu") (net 16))
 (segment (start 192.23 88.77) (end 196.5 84.5) (width 0.4) (layer "F.Cu") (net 16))
 (segment (start 188.8 67.3) (end 140 67.3) (width 0.4) (layer "F.Cu") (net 16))
 (segment (start 154 99.5) (end 145.2 108.3) (width 0.4) (layer "F.Cu") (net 5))
 (segment (start 160.23 88.77) (end 154 95) (width 0.4) (layer "F.Cu") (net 5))
 (segment (start 154 95) (end 154 99.5) (width 0.4) (layer "F.Cu") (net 5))
 (segment (start 145.2 108.3) (end 140 108.3) (width 0.4) (layer "F.Cu") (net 5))
 (segment (start 182.785 88.77) (end 160.23 88.77) (width 0.4) (layer "F.Cu") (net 5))
 (segment (start 195 84) (end 191.5 87.5) (width 0.4) (layer "F.Cu") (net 17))
 (segment (start 188.84 69.84) (end 195 76) (width 0.4) (layer "F.Cu") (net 17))
 (segment (start 191.5 87.5) (end 186.215 87.5) (width 0.4) (layer "F.Cu") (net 17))
 (segment (start 140 69.84) (end 188.84 69.84) (width 0.4) (layer "F.Cu") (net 17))
 (segment (start 195 76) (end 195 84) (width 0.4) (layer "F.Cu") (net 17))
 (segment (start 190.77 86.23) (end 193.5 83.5) (width 0.4) (layer "F.Cu") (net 18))
 (segment (start 188.88 72.38) (end 140 72.38) (width 0.4) (layer "F.Cu") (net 18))
 (segment (start 193.5 77) (end 188.88 72.38) (width 0.4) (layer "F.Cu") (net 18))
 (segment (start 186.215 86.23) (end 190.77 86.23) (width 0.4) (layer "F.Cu") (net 18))
 (segment (start 193.5 83.5) (end 193.5 77) (width 0.4) (layer "F.Cu") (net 18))
 (segment (start 150 93) (end 150 98.5) (width 0.4) (layer "F.Cu") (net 3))
 (segment (start 150 98.5) (end 145.28 103.22) (width 0.4) (layer "F.Cu") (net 3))
 (segment (start 145.28 103.22) (end 140 103.22) (width 0.4) (layer "F.Cu") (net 3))
 (segment (start 156.77 86.23) (end 150 93) (width 0.4) (layer "F.Cu") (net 3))
 (segment (start 182.785 86.23) (end 156.77 86.23) (width 0.4) (layer "F.Cu") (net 3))
 (segment (start 192 82.96) (end 190 84.96) (width 0.4) (layer "F.Cu") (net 19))
 (segment (start 190 84.96) (end 186.215 84.96) (width 0.4) (layer "F.Cu") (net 19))
 (segment (start 140 74.92) (end 189.42 74.92) (width 0.4) (layer "F.Cu") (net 19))
 (segment (start 192 77.5) (end 192 82.96) (width 0.4) (layer "F.Cu") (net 19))
 (segment (start 189.42 74.92) (end 192 77.5) (width 0.4) (layer "F.Cu") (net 19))
 (segment (start 140 100.68) (end 145.32 100.68) (width 0.4) (layer "F.Cu") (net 2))
 (segment (start 145.32 100.68) (end 148 98) (width 0.4) (layer "F.Cu") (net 2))
 (segment (start 148 92.5) (end 155.54 84.96) (width 0.4) (layer "F.Cu") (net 2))
 (segment (start 155.54 84.96) (end 182.785 84.96) (width 0.4) (layer "F.Cu") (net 2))
 (segment (start 148 98) (end 148 92.5) (width 0.4) (layer "F.Cu") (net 2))
 (segment (start 190.5 82.5) (end 190.5 78.5) (width 0.4) (layer "F.Cu") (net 20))
 (segment (start 189.46 77.46) (end 140 77.46) (width 0.4) (layer "F.Cu") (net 20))
 (segment (start 190.5 78.5) (end 189.46 77.46) (width 0.4) (layer "F.Cu") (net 20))
 (segment (start 186.215 83.69) (end 189.31 83.69) (width 0.4) (layer "F.Cu") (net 20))
 (segment (start 189.31 83.69) (end 190.5 82.5) (width 0.4) (layer "F.Cu") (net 20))
 (segment (start 146.5 97) (end 145.36 98.14) (width 0.4) (layer "F.Cu") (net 1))
 (segment (start 146.5 91.5) (end 146.5 97) (width 0.4) (layer "F.Cu") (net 1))
 (segment (start 154.31 83.69) (end 146.5 91.5) (width 0.4) (layer "F.Cu") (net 1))
 (segment (start 145.36 98.14) (end 140 98.14) (width 0.4) (layer "F.Cu") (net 1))
 (segment (start 182.785 83.69) (end 154.31 83.69) (width 0.4) (layer "F.Cu") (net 1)))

